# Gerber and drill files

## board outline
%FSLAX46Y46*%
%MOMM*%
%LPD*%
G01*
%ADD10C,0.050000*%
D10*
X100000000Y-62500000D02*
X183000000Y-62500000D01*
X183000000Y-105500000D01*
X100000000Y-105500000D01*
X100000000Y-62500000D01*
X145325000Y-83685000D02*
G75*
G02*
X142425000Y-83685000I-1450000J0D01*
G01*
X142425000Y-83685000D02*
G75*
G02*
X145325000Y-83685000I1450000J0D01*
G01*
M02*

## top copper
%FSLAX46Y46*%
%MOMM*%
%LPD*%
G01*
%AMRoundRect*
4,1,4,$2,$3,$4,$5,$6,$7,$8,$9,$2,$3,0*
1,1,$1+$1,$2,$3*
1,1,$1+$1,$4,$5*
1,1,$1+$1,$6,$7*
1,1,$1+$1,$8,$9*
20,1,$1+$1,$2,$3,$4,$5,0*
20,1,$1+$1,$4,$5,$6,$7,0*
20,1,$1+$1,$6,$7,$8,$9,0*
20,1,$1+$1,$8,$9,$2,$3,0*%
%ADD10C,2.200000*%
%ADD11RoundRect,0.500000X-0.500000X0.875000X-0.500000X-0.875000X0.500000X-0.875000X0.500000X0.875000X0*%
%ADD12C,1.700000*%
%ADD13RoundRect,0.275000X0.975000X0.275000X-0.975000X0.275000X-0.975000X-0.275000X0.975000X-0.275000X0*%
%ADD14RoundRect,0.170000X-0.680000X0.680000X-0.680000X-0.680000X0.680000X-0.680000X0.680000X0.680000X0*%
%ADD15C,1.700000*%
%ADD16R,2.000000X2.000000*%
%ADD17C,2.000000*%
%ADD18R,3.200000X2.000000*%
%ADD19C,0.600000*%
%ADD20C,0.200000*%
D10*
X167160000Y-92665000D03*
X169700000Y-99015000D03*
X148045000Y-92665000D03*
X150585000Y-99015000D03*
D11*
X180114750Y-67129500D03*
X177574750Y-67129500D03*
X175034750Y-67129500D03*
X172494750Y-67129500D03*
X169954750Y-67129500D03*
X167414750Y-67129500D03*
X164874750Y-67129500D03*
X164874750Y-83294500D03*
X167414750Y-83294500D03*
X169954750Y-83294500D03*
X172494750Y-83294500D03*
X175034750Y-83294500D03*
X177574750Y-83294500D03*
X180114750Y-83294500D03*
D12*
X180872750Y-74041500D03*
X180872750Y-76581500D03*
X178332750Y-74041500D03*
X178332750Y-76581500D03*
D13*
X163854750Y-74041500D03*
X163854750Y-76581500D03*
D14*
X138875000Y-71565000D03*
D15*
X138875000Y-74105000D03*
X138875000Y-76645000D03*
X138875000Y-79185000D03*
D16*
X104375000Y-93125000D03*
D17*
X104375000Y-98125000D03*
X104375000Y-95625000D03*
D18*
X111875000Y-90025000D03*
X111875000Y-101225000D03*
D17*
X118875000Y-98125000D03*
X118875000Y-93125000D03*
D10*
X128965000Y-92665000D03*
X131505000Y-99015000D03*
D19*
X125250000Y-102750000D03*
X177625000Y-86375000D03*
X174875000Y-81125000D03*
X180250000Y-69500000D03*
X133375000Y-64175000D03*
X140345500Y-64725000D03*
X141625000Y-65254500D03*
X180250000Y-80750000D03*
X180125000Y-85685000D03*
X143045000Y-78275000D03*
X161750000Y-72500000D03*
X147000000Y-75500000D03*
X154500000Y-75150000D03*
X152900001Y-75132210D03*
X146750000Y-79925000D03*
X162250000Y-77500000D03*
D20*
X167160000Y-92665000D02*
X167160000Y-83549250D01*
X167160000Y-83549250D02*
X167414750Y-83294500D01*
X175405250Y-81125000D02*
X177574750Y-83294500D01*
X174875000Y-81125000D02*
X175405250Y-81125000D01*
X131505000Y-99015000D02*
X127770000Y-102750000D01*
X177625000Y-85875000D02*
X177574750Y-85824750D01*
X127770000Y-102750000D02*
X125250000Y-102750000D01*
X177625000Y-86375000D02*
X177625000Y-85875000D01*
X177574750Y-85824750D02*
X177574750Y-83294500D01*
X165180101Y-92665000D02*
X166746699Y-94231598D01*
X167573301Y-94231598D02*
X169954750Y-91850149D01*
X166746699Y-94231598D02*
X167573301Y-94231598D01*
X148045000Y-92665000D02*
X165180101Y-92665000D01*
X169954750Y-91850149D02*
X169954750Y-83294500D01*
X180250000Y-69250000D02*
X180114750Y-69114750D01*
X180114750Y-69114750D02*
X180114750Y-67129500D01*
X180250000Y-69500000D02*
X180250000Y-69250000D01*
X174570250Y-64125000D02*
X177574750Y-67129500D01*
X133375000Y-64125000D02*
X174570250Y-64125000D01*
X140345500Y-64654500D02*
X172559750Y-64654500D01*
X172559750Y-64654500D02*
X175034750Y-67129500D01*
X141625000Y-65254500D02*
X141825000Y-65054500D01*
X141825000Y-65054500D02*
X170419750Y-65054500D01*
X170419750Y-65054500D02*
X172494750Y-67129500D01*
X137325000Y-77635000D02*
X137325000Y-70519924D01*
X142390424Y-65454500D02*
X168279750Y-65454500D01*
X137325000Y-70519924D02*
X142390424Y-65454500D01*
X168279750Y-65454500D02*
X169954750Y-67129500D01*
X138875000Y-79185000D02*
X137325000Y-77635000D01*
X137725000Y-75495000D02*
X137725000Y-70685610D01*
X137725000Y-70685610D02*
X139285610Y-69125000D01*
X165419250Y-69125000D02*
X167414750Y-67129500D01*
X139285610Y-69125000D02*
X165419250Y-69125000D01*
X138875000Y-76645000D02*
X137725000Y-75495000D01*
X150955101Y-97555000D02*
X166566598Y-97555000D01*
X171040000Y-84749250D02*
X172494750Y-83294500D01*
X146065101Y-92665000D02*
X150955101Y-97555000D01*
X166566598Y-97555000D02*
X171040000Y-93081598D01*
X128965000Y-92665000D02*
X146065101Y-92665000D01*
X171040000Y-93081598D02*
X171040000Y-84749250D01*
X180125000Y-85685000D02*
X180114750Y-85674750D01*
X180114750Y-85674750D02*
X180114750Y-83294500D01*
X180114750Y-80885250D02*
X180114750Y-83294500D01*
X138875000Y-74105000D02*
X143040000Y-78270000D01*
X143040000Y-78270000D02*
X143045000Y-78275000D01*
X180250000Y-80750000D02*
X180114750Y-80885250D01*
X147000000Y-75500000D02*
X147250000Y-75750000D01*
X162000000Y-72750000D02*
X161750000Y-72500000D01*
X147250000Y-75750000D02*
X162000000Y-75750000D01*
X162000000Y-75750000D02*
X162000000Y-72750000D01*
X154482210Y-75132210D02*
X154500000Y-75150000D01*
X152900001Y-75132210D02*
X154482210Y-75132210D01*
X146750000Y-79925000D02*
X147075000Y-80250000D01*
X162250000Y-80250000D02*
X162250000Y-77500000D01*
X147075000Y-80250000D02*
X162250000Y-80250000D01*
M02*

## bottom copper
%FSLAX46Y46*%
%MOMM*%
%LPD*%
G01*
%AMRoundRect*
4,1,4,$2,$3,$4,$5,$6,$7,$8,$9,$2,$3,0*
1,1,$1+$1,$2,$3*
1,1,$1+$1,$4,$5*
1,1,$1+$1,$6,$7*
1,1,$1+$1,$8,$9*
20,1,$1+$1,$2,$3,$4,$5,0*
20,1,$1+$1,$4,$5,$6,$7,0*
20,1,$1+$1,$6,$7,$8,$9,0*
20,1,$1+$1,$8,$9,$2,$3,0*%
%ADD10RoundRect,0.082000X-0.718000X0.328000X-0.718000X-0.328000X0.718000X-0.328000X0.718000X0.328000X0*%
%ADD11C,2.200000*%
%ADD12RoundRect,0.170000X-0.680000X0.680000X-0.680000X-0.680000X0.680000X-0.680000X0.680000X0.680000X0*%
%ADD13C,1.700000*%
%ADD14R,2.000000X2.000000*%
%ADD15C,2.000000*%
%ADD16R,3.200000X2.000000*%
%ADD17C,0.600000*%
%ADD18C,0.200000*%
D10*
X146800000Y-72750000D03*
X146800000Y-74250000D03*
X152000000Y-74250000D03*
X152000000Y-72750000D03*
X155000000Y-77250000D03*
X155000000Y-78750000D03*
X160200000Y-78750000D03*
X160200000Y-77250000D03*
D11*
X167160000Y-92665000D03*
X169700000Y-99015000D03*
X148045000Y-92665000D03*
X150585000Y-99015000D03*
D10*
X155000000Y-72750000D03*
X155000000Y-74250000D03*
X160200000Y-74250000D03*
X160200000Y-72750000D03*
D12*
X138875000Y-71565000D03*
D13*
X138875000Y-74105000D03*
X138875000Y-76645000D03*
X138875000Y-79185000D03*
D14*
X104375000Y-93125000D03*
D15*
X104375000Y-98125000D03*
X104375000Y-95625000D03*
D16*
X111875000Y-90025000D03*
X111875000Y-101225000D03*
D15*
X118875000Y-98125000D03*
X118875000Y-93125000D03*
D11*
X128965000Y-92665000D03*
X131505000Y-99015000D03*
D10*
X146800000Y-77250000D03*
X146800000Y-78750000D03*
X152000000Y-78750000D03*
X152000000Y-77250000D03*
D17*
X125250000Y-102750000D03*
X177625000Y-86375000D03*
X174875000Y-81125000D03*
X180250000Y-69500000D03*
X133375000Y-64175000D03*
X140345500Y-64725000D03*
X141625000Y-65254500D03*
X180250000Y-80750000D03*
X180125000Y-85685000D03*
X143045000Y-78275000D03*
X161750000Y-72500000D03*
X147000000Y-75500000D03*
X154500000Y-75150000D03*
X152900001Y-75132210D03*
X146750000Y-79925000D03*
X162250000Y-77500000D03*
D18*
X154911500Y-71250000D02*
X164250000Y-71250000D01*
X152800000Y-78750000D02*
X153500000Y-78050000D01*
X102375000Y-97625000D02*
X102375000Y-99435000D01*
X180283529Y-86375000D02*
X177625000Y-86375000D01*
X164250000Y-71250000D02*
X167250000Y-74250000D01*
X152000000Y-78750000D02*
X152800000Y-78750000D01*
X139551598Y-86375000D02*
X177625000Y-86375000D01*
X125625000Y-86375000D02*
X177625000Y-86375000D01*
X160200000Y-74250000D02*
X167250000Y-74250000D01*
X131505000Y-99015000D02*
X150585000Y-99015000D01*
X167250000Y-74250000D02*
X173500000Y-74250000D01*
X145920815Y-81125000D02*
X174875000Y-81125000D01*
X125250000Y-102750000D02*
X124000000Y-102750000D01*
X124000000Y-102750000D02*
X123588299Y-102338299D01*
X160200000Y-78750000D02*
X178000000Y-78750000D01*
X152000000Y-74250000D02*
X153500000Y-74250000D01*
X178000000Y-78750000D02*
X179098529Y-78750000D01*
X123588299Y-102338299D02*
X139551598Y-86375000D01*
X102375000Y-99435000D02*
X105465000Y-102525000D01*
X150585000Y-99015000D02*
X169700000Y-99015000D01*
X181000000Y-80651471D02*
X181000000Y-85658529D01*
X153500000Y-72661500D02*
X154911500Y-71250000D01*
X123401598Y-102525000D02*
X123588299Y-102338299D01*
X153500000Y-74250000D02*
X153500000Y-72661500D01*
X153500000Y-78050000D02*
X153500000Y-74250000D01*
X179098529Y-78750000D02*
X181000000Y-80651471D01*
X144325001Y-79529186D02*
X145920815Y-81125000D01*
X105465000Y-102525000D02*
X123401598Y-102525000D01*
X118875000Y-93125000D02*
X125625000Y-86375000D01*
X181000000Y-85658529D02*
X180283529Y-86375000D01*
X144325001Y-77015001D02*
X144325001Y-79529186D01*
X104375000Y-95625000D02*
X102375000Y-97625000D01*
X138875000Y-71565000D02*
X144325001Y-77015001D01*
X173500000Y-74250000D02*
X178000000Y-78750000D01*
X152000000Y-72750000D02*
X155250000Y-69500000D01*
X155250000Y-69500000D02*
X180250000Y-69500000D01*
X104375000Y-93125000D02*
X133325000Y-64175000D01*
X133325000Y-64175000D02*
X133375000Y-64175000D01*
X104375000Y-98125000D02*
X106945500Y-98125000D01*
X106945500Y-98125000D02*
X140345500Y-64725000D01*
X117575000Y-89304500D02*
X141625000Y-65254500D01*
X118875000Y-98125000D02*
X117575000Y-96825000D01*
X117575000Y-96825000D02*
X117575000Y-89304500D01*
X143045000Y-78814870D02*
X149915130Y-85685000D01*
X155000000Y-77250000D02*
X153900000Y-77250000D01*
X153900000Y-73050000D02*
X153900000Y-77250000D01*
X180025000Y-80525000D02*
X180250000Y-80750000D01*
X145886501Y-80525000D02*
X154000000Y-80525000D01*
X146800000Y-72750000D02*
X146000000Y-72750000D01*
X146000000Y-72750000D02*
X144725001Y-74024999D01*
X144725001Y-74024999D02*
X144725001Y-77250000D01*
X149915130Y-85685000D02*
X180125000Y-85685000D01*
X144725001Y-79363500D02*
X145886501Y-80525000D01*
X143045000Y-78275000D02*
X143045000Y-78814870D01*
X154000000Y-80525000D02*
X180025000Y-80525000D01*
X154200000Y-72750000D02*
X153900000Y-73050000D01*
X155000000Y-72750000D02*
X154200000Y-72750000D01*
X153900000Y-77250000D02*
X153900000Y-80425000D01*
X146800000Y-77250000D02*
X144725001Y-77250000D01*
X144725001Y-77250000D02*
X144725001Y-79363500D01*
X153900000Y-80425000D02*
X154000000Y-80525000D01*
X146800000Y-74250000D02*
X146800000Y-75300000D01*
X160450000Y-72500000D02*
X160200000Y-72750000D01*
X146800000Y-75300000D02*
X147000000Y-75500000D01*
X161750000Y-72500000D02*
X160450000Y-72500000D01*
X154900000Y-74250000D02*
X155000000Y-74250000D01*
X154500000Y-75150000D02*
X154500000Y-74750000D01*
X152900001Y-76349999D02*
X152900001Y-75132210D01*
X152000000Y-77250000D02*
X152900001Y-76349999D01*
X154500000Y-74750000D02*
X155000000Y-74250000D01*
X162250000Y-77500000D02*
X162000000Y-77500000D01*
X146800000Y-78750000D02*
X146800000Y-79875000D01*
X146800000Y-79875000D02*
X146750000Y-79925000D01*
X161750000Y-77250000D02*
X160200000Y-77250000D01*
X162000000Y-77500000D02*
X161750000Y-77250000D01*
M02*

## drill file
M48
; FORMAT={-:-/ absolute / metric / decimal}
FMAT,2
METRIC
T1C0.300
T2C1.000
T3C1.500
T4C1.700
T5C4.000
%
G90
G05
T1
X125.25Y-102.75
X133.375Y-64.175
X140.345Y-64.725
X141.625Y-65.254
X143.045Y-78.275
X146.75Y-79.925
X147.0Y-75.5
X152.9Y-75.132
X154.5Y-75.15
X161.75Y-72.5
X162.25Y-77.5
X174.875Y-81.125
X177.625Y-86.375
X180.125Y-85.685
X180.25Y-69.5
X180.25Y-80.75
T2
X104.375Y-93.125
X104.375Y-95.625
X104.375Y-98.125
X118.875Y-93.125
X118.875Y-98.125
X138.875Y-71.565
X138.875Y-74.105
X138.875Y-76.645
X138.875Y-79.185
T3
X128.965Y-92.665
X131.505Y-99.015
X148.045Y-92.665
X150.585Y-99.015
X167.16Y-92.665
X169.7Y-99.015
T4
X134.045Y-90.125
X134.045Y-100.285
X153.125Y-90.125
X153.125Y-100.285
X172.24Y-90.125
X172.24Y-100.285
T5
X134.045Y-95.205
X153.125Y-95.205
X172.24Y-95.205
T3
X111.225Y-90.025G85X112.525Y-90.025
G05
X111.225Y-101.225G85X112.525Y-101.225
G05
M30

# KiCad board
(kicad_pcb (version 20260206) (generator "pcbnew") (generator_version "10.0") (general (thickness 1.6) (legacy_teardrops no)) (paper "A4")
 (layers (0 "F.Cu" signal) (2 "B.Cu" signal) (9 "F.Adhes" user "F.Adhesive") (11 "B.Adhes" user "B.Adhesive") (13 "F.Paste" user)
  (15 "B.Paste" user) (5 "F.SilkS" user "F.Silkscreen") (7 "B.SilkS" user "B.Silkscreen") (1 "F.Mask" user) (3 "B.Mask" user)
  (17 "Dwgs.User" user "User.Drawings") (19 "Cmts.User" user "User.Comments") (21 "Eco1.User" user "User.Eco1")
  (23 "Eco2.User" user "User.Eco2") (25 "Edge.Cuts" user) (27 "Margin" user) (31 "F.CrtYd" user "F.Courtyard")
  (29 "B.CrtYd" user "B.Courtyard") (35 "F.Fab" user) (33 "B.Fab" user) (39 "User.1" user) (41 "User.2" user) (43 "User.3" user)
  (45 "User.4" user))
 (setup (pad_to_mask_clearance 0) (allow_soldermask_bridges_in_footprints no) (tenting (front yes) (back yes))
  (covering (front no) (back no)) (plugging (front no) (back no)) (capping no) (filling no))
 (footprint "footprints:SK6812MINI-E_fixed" (layer "F.Cu") (at 149.399999 73.602842)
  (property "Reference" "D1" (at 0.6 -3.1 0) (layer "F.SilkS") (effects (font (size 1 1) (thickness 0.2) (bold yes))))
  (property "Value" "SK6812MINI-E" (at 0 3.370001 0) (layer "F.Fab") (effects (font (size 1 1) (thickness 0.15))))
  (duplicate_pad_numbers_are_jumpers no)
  (pad "1" smd roundrect (at -2.599999 -0.852842 270) (size 0.82 1.6) (layers "B.Cu" "B.Mask" "B.Paste") (roundrect_rratio 0.1) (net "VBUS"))
  (pad "2" smd roundrect (at -2.599999 0.647158 270) (size 0.82 1.6) (layers "B.Cu" "B.Mask" "B.Paste") (roundrect_rratio 0.1)
   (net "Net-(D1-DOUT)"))
  (pad "3" smd roundrect (at 2.600001 0.647158 270) (size 0.82 1.6) (layers "B.Cu" "B.Mask" "B.Paste") (roundrect_rratio 0.1) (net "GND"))
  (pad "4" smd roundrect (at 2.600001 -0.852842 270) (size 0.82 1.6) (layers "B.Cu" "B.Mask" "B.Paste") (roundrect_rratio 0.1)
   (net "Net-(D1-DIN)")))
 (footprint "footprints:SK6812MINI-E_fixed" (layer "F.Cu") (at 157.599999 78.102842)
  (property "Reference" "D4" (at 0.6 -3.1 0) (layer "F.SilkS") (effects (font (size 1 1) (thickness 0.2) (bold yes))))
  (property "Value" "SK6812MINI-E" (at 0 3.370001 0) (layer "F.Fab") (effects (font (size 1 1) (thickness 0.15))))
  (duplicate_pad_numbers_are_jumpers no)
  (pad "1" smd roundrect (at -2.599999 -0.852842 270) (size 0.82 1.6) (layers "B.Cu" "B.Mask" "B.Paste") (roundrect_rratio 0.1) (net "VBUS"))
  (pad "2" smd roundrect (at -2.599999 0.647158 270) (size 0.82 1.6) (layers "B.Cu" "B.Mask" "B.Paste") (roundrect_rratio 0.1)
   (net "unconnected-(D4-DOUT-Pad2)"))
  (pad "3" smd roundrect (at 2.600001 0.647158 270) (size 0.82 1.6) (layers "B.Cu" "B.Mask" "B.Paste") (roundrect_rratio 0.1) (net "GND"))
  (pad "4" smd roundrect (at 2.600001 -0.852842 270) (size 0.82 1.6) (layers "B.Cu" "B.Mask" "B.Paste") (roundrect_rratio 0.1)
   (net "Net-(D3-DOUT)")))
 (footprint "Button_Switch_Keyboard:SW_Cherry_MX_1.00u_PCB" (layer "F.Cu") (at 167.16 92.665 90)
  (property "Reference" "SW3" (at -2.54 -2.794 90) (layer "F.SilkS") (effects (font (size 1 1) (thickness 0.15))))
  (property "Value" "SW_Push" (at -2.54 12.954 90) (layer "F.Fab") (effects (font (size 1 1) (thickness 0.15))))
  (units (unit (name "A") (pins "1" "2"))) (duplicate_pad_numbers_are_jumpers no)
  (pad "" np_thru_hole circle (at -7.62 5.08 90) (size 1.7 1.7) (drill 1.7) (layers "*.Cu" "*.Mask"))
  (pad "" np_thru_hole circle (at -2.54 5.08 90) (size 4 4) (drill 4) (layers "*.Cu" "*.Mask"))
  (pad "" np_thru_hole circle (at 2.54 5.08 90) (size 1.7 1.7) (drill 1.7) (layers "*.Cu" "*.Mask"))
  (pad "1" thru_hole circle (at 0 0 90) (size 2.2 2.2) (drill 1.5) (layers "*.Cu" "*.Mask") (remove_unused_layers no) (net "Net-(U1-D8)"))
  (pad "2" thru_hole circle (at -6.35 2.54 90) (size 2.2 2.2) (drill 1.5) (layers "*.Cu" "*.Mask") (remove_unused_layers no) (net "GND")))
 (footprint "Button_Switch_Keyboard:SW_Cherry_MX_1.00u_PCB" (layer "F.Cu") (at 148.045 92.665 90)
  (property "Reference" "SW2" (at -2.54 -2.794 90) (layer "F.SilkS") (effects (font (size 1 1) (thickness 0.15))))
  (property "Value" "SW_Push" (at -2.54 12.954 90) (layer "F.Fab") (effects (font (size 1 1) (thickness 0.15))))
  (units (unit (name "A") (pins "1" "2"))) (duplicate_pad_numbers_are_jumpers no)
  (pad "" np_thru_hole circle (at -7.62 5.08 90) (size 1.7 1.7) (drill 1.7) (layers "*.Cu" "*.Mask"))
  (pad "" np_thru_hole circle (at -2.54 5.08 90) (size 4 4) (drill 4) (layers "*.Cu" "*.Mask"))
  (pad "" np_thru_hole circle (at 2.54 5.08 90) (size 1.7 1.7) (drill 1.7) (layers "*.Cu" "*.Mask"))
  (pad "1" thru_hole circle (at 0 0 90) (size 2.2 2.2) (drill 1.5) (layers "*.Cu" "*.Mask") (remove_unused_layers no) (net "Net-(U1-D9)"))
  (pad "2" thru_hole circle (at -6.35 2.54 90) (size 2.2 2.2) (drill 1.5) (layers "*.Cu" "*.Mask") (remove_unused_layers no) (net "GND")))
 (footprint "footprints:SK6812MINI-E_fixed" (layer "F.Cu") (at 157.599999 73.602842)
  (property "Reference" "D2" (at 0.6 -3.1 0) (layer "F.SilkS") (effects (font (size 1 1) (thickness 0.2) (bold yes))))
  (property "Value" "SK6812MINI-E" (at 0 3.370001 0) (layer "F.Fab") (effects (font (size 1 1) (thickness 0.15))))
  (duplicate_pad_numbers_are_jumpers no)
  (pad "1" smd roundrect (at -2.599999 -0.852842 270) (size 0.82 1.6) (layers "B.Cu" "B.Mask" "B.Paste") (roundrect_rratio 0.1) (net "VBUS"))
  (pad "2" smd roundrect (at -2.599999 0.647158 270) (size 0.82 1.6) (layers "B.Cu" "B.Mask" "B.Paste") (roundrect_rratio 0.1)
   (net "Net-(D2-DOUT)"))
  (pad "3" smd roundrect (at 2.600001 0.647158 270) (size 0.82 1.6) (layers "B.Cu" "B.Mask" "B.Paste") (roundrect_rratio 0.1) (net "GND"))
  (pad "4" smd roundrect (at 2.600001 -0.852842 270) (size 0.82 1.6) (layers "B.Cu" "B.Mask" "B.Paste") (roundrect_rratio 0.1)
   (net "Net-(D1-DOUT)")))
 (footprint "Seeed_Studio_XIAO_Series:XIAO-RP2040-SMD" (layer "F.Cu") (at 161.99475 66.2945 -90)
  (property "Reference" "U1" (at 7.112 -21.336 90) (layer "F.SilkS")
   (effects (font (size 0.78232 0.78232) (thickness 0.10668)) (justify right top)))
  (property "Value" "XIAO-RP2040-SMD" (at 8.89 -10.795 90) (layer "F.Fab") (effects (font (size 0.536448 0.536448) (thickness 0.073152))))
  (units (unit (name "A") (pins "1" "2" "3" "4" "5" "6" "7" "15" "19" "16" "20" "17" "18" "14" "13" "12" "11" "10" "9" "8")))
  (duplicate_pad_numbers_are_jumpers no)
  (pad "1" smd roundrect (at 0.835 -18.12 270) (size 2.75 2) (layers "F.Cu" "F.Mask" "F.Paste") (roundrect_rratio 0.25) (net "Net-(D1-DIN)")
   (solder_mask_margin 0.0508) (thermal_bridge_angle 45))
  (pad "2" smd roundrect (at 0.835 -15.58 270) (size 2.75 2) (layers "F.Cu" "F.Mask" "F.Paste") (roundrect_rratio 0.25) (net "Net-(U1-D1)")
   (solder_mask_margin 0.0508) (thermal_bridge_angle 45))
  (pad "3" smd roundrect (at 0.835 -13.04 270) (size 2.75 2) (layers "F.Cu" "F.Mask" "F.Paste") (roundrect_rratio 0.25) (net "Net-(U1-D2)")
   (solder_mask_margin 0.0508) (thermal_bridge_angle 45))
  (pad "4" smd roundrect (at 0.835 -10.5 270) (size 2.75 2) (layers "F.Cu" "F.Mask" "F.Paste") (roundrect_rratio 0.25) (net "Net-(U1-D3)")
   (solder_mask_margin 0.0508) (thermal_bridge_angle 45))
  (pad "5" smd roundrect (at 0.835 -7.96 270) (size 2.75 2) (layers "F.Cu" "F.Mask" "F.Paste") (roundrect_rratio 0.25) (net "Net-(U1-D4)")
   (solder_mask_margin 0.0508) (thermal_bridge_angle 45))
  (pad "6" smd roundrect (at 0.835 -5.42 270) (size 2.75 2) (layers "F.Cu" "F.Mask" "F.Paste") (roundrect_rratio 0.25) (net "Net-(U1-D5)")
   (solder_mask_margin 0.0508) (thermal_bridge_angle 45))
  (pad "7" smd roundrect (at 0.835 -2.88 270) (size 2.75 2) (layers "F.Cu" "F.Mask" "F.Paste") (roundrect_rratio 0.25)
   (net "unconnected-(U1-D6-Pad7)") (solder_mask_margin 0.0508) (thermal_bridge_angle 45))
  (pad "8" smd roundrect (at 17 -2.88 270) (size 2.75 2) (layers "F.Cu" "F.Mask" "F.Paste") (roundrect_rratio 0.25)
   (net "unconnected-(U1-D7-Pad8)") (solder_mask_margin 0.0508) (thermal_bridge_angle 45))
  (pad "9" smd roundrect (at 17 -5.42 270) (size 2.75 2) (layers "F.Cu" "F.Mask" "F.Paste") (roundrect_rratio 0.25) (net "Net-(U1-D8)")
   (solder_mask_margin 0.0508) (thermal_bridge_angle 45))
  (pad "10" smd roundrect (at 17 -7.96 270) (size 2.75 2) (layers "F.Cu" "F.Mask" "F.Paste") (roundrect_rratio 0.25) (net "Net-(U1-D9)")
   (solder_mask_margin 0.0508) (thermal_bridge_angle 45))
  (pad "11" smd roundrect (at 17 -10.5 270) (size 2.75 2) (layers "F.Cu" "F.Mask" "F.Paste") (roundrect_rratio 0.25) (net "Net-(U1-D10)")
   (solder_mask_margin 0.0508) (thermal_bridge_angle 45))
  (pad "12" smd roundrect (at 17 -13.04 270) (size 2.75 2) (layers "F.Cu" "F.Mask" "F.Paste") (roundrect_rratio 0.25)
   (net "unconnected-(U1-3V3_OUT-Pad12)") (solder_mask_margin 0.0508) (thermal_bridge_angle 45))
  (pad "13" smd roundrect (at 17 -15.58 270) (size 2.75 2) (layers "F.Cu" "F.Mask" "F.Paste") (roundrect_rratio 0.25) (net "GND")
   (solder_mask_margin 0.0508) (thermal_bridge_angle 45))
  (pad "14" smd roundrect (at 17 -18.12 270) (size 2.75 2) (layers "F.Cu" "F.Mask" "F.Paste") (roundrect_rratio 0.25) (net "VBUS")
   (solder_mask_margin 0.0508) (thermal_bridge_angle 45))
  (pad "15" smd circle (at 7.747 -18.878 270) (size 1.7 1.7) (layers "F.Cu" "F.Mask" "F.Paste") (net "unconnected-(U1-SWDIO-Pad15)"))
  (pad "16" smd circle (at 10.287 -18.878 270) (size 1.7 1.7) (layers "F.Cu" "F.Mask" "F.Paste") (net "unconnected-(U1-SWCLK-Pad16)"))
  (pad "17" smd circle (at 7.747 -16.338 270) (size 1.7 1.7) (layers "F.Cu" "F.Mask" "F.Paste") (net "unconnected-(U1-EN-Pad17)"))
  (pad "18" smd circle (at 10.287 -16.338 270) (size 1.7 1.7) (layers "F.Cu" "F.Mask" "F.Paste") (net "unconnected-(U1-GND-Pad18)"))
  (pad "19" smd roundrect (at 7.747 -1.86 180) (size 2.5 1.1) (layers "F.Cu" "F.Mask" "F.Paste") (roundrect_rratio 0.25)
   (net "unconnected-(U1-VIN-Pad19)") (thermal_bridge_angle 45))
  (pad "20" smd roundrect (at 10.287 -1.86 180) (size 2.5 1.1) (layers "F.Cu" "F.Mask" "F.Paste") (roundrect_rratio 0.25)
   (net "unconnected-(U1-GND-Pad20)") (thermal_bridge_angle 45)))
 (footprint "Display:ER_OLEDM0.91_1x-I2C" (layer "F.Cu") (at 138.875 71.565 -90)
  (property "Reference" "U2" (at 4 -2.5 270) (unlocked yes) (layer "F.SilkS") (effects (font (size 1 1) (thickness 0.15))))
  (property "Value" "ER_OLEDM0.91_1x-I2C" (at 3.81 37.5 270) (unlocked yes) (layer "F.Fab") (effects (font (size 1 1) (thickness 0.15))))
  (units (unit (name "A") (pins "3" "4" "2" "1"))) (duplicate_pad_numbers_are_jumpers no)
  (pad "1" thru_hole roundrect (at 0 0 270) (size 1.7 1.7) (drill 1) (layers "*.Cu" "*.Mask") (remove_unused_layers no)
   (roundrect_rratio 0.1) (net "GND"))
  (pad "2" thru_hole circle (at 2.54 0 270) (size 1.7 1.7) (drill 1) (layers "*.Cu" "*.Mask") (remove_unused_layers no) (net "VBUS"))
  (pad "3" thru_hole circle (at 5.08 0 270) (size 1.7 1.7) (drill 1) (layers "*.Cu" "*.Mask") (remove_unused_layers no) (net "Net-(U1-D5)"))
  (pad "4" thru_hole circle (at 7.62 0 270) (size 1.7 1.7) (drill 1) (layers "*.Cu" "*.Mask") (remove_unused_layers no) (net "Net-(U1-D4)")))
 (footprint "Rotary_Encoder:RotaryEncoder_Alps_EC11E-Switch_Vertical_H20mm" (layer "F.Cu") (at 104.375 93.125)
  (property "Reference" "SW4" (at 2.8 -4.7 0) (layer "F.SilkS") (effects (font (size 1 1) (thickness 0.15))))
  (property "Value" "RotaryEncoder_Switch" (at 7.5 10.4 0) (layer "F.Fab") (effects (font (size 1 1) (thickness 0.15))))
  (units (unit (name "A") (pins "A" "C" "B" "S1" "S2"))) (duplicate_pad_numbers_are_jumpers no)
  (pad "A" thru_hole rect (at 0 0) (size 2 2) (drill 1) (layers "*.Cu" "*.Mask") (remove_unused_layers no) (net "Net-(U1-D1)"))
  (pad "B" thru_hole circle (at 0 5) (size 2 2) (drill 1) (layers "*.Cu" "*.Mask") (remove_unused_layers no) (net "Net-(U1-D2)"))
  (pad "C" thru_hole circle (at 0 2.5) (size 2 2) (drill 1) (layers "*.Cu" "*.Mask") (remove_unused_layers no) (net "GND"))
  (pad "MP" thru_hole rect (at 7.5 -3.1) (size 3.2 2) (drill oval 2.8 1.5) (layers "*.Cu" "*.Mask") (remove_unused_layers no))
  (pad "MP" thru_hole rect (at 7.5 8.1) (size 3.2 2) (drill oval 2.8 1.5) (layers "*.Cu" "*.Mask") (remove_unused_layers no))
  (pad "S1" thru_hole circle (at 14.5 5) (size 2 2) (drill 1) (layers "*.Cu" "*.Mask") (remove_unused_layers no) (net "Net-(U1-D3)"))
  (pad "S2" thru_hole circle (at 14.5 0) (size 2 2) (drill 1) (layers "*.Cu" "*.Mask") (remove_unused_layers no) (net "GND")))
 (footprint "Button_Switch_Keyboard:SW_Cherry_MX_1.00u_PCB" (layer "F.Cu") (at 128.965 92.665 90)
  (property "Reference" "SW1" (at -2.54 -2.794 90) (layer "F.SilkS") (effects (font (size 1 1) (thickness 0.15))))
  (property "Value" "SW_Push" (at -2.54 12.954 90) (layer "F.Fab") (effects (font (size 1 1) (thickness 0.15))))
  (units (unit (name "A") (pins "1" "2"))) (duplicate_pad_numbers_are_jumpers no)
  (pad "" np_thru_hole circle (at -7.62 5.08 90) (size 1.7 1.7) (drill 1.7) (layers "*.Cu" "*.Mask"))
  (pad "" np_thru_hole circle (at -2.54 5.08 90) (size 4 4) (drill 4) (layers "*.Cu" "*.Mask"))
  (pad "" np_thru_hole circle (at 2.54 5.08 90) (size 1.7 1.7) (drill 1.7) (layers "*.Cu" "*.Mask"))
  (pad "1" thru_hole circle (at 0 0 90) (size 2.2 2.2) (drill 1.5) (layers "*.Cu" "*.Mask") (remove_unused_layers no) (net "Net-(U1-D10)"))
  (pad "2" thru_hole circle (at -6.35 2.54 90) (size 2.2 2.2) (drill 1.5) (layers "*.Cu" "*.Mask") (remove_unused_layers no) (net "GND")))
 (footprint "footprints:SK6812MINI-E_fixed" (layer "F.Cu") (at 149.399999 78.102842)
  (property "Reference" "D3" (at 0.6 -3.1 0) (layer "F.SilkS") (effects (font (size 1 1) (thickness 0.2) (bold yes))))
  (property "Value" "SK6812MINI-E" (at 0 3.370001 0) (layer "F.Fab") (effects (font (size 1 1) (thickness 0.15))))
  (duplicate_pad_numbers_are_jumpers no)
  (pad "1" smd roundrect (at -2.599999 -0.852842 270) (size 0.82 1.6) (layers "B.Cu" "B.Mask" "B.Paste") (roundrect_rratio 0.1) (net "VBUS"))
  (pad "2" smd roundrect (at -2.599999 0.647158 270) (size 0.82 1.6) (layers "B.Cu" "B.Mask" "B.Paste") (roundrect_rratio 0.1)
   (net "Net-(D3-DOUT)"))
  (pad "3" smd roundrect (at 2.600001 0.647158 270) (size 0.82 1.6) (layers "B.Cu" "B.Mask" "B.Paste") (roundrect_rratio 0.1) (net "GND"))
  (pad "4" smd roundrect (at 2.600001 -0.852842 270) (size 0.82 1.6) (layers "B.Cu" "B.Mask" "B.Paste") (roundrect_rratio 0.1)
   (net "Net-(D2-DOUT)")))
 (gr_rect (start 100 62.5) (end 183 105.5) (stroke (width 0.05) (type solid)) (fill no) (layer "Edge.Cuts"))
 (gr_circle (center 143.875 83.685) (end 145.325 83.685) (stroke (width 0.05) (type default)) (fill no) (layer "Edge.Cuts"))
 (segment (start 167.16 92.665) (end 167.16 83.54925) (width 0.2) (layer "F.Cu") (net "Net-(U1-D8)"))
 (segment (start 167.16 83.54925) (end 167.41475 83.2945) (width 0.2) (layer "F.Cu") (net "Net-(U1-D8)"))
 (segment (start 175.40525 81.125) (end 177.57475 83.2945) (width 0.2) (layer "F.Cu") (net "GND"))
 (segment (start 174.875 81.125) (end 175.40525 81.125) (width 0.2) (layer "F.Cu") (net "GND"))
 (segment (start 131.505 99.015) (end 127.77 102.75) (width 0.2) (layer "F.Cu") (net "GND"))
 (segment (start 177.625 85.875) (end 177.57475 85.82475) (width 0.2) (layer "F.Cu") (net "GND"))
 (segment (start 127.77 102.75) (end 125.25 102.75) (width 0.2) (layer "F.Cu") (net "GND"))
 (segment (start 177.625 86.375) (end 177.625 85.875) (width 0.2) (layer "F.Cu") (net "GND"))
 (segment (start 177.57475 85.82475) (end 177.57475 83.2945) (width 0.2) (layer "F.Cu") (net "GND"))
 (via (at 125.25 102.75) (size 0.6) (drill 0.3) (layers "F.Cu" "B.Cu") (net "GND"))
 (via (at 177.625 86.375) (size 0.6) (drill 0.3) (layers "F.Cu" "B.Cu") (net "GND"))
 (via (at 174.875 81.125) (size 0.6) (drill 0.3) (layers "F.Cu" "B.Cu") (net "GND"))
 (segment (start 154.9115 71.25) (end 164.25 71.25) (width 0.2) (layer "B.Cu") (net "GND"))
 (segment (start 152.8 78.75) (end 153.5 78.05) (width 0.2) (layer "B.Cu") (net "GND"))
 (segment (start 102.375 97.625) (end 102.375 99.435) (width 0.2) (layer "B.Cu") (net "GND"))
 (segment (start 180.283529 86.375) (end 177.625 86.375) (width 0.2) (layer "B.Cu") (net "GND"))
 (segment (start 164.25 71.25) (end 167.25 74.25) (width 0.2) (layer "B.Cu") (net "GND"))
 (segment (start 152 78.75) (end 152.8 78.75) (width 0.2) (layer "B.Cu") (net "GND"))
 (segment (start 139.551598 86.375) (end 177.625 86.375) (width 0.2) (layer "B.Cu") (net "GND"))
 (segment (start 125.625 86.375) (end 177.625 86.375) (width 0.2) (layer "B.Cu") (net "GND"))
 (segment (start 160.2 74.25) (end 167.25 74.25) (width 0.2) (layer "B.Cu") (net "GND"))
 (segment (start 131.505 99.015) (end 150.585 99.015) (width 0.2) (layer "B.Cu") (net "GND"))
 (segment (start 167.25 74.25) (end 173.5 74.25) (width 0.2) (layer "B.Cu") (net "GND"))
 (segment (start 145.920815 81.125) (end 174.875 81.125) (width 0.2) (layer "B.Cu") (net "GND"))
 (segment (start 125.25 102.75) (end 124 102.75) (width 0.2) (layer "B.Cu") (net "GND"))
 (segment (start 124 102.75) (end 123.588299 102.338299) (width 0.2) (layer "B.Cu") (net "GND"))
 (segment (start 160.2 78.75) (end 178 78.75) (width 0.2) (layer "B.Cu") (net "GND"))
 (segment (start 152 74.25) (end 153.5 74.25) (width 0.2) (layer "B.Cu") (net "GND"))
 (segment (start 178 78.75) (end 179.098529 78.75) (width 0.2) (layer "B.Cu") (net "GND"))
 (segment (start 123.588299 102.338299) (end 139.551598 86.375) (width 0.2) (layer "B.Cu") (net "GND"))
 (segment (start 102.375 99.435) (end 105.465 102.525) (width 0.2) (layer "B.Cu") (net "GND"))
 (segment (start 150.585 99.015) (end 169.7 99.015) (width 0.2) (layer "B.Cu") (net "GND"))
 (segment (start 181 80.651471) (end 181 85.658529) (width 0.2) (layer "B.Cu") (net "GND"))
 (segment (start 153.5 72.6615) (end 154.9115 71.25) (width 0.2) (layer "B.Cu") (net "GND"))
 (segment (start 123.401598 102.525) (end 123.588299 102.338299) (width 0.2) (layer "B.Cu") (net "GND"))
 (segment (start 153.5 74.25) (end 153.5 72.6615) (width 0.2) (layer "B.Cu") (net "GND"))
 (segment (start 153.5 78.05) (end 153.5 74.25) (width 0.2) (layer "B.Cu") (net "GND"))
 (segment (start 179.098529 78.75) (end 181 80.651471) (width 0.2) (layer "B.Cu") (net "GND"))
 (segment (start 144.325001 79.529186) (end 145.920815 81.125) (width 0.2) (layer "B.Cu") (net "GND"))
 (segment (start 105.465 102.525) (end 123.401598 102.525) (width 0.2) (layer "B.Cu") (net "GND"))
 (segment (start 118.875 93.125) (end 125.625 86.375) (width 0.2) (layer "B.Cu") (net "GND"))
 (segment (start 181 85.658529) (end 180.283529 86.375) (width 0.2) (layer "B.Cu") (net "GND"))
 (segment (start 144.325001 77.015001) (end 144.325001 79.529186) (width 0.2) (layer "B.Cu") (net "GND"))
 (segment (start 104.375 95.625) (end 102.375 97.625) (width 0.2) (layer "B.Cu") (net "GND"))
 (segment (start 138.875 71.565) (end 144.325001 77.015001) (width 0.2) (layer "B.Cu") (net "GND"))
 (segment (start 173.5 74.25) (end 178 78.75) (width 0.2) (layer "B.Cu") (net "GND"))
 (segment (start 165.180101 92.665) (end 166.746699 94.231598) (width 0.2) (layer "F.Cu") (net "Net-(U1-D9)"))
 (segment (start 167.573301 94.231598) (end 169.95475 91.850149) (width 0.2) (layer "F.Cu") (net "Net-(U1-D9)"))
 (segment (start 166.746699 94.231598) (end 167.573301 94.231598) (width 0.2) (layer "F.Cu") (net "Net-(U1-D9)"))
 (segment (start 148.045 92.665) (end 165.180101 92.665) (width 0.2) (layer "F.Cu") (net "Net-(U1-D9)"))
 (segment (start 169.95475 91.850149) (end 169.95475 83.2945) (width 0.2) (layer "F.Cu") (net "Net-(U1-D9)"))
 (segment (start 180.25 69.25) (end 180.11475 69.11475) (width 0.2) (layer "F.Cu") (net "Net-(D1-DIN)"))
 (segment (start 180.11475 69.11475) (end 180.11475 67.1295) (width 0.2) (layer "F.Cu") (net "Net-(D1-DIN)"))
 (segment (start 180.25 69.5) (end 180.25 69.25) (width 0.2) (layer "F.Cu") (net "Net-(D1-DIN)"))
 (via (at 180.25 69.5) (size 0.6) (drill 0.3) (layers "F.Cu" "B.Cu") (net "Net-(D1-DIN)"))
 (segment (start 152 72.75) (end 155.25 69.5) (width 0.2) (layer "B.Cu") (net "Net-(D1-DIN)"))
 (segment (start 155.25 69.5) (end 180.25 69.5) (width 0.2) (layer "B.Cu") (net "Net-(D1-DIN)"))
 (segment (start 174.57025 64.125) (end 177.57475 67.1295) (width 0.2) (layer "F.Cu") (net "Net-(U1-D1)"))
 (segment (start 133.375 64.125) (end 174.57025 64.125) (width 0.2) (layer "F.Cu") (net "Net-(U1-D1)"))
 (via (at 133.375 64.175) (size 0.6) (drill 0.3) (layers "F.Cu" "B.Cu") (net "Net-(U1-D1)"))
 (segment (start 104.375 93.125) (end 133.325 64.175) (width 0.2) (layer "B.Cu") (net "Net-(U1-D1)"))
 (segment (start 133.325 64.175) (end 133.375 64.175) (width 0.2) (layer "B.Cu") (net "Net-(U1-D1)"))
 (segment (start 140.3455 64.6545) (end 172.55975 64.6545) (width 0.2) (layer "F.Cu") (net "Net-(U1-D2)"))
 (segment (start 172.55975 64.6545) (end 175.03475 67.1295) (width 0.2) (layer "F.Cu") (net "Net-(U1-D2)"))
 (via (at 140.3455 64.725) (size 0.6) (drill 0.3) (layers "F.Cu" "B.Cu") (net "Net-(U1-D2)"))
 (segment (start 104.375 98.125) (end 106.9455 98.125) (width 0.2) (layer "B.Cu") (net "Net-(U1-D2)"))
 (segment (start 106.9455 98.125) (end 140.3455 64.725) (width 0.2) (layer "B.Cu") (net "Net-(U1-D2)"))
 (segment (start 141.625 65.2545) (end 141.825 65.0545) (width 0.2) (layer "F.Cu") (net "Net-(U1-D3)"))
 (segment (start 141.825 65.0545) (end 170.41975 65.0545) (width 0.2) (layer "F.Cu") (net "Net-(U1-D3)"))
 (segment (start 170.41975 65.0545) (end 172.49475 67.1295) (width 0.2) (layer "F.Cu") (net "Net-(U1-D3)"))
 (via (at 141.625 65.2545) (size 0.6) (drill 0.3) (layers "F.Cu" "B.Cu") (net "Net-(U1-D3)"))
 (segment (start 117.575 89.3045) (end 141.625 65.2545) (width 0.2) (layer "B.Cu") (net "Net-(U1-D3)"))
 (segment (start 118.875 98.125) (end 117.575 96.825) (width 0.2) (layer "B.Cu") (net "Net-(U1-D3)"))
 (segment (start 117.575 96.825) (end 117.575 89.3045) (width 0.2) (layer "B.Cu") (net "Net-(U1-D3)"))
 (segment (start 137.325 77.635) (end 137.325 70.519924) (width 0.2) (layer "F.Cu") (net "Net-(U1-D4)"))
 (segment (start 142.390424 65.4545) (end 168.27975 65.4545) (width 0.2) (layer "F.Cu") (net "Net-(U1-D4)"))
 (segment (start 137.325 70.519924) (end 142.390424 65.4545) (width 0.2) (layer "F.Cu") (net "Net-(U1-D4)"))
 (segment (start 168.27975 65.4545) (end 169.95475 67.1295) (width 0.2) (layer "F.Cu") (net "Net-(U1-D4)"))
 (segment (start 138.875 79.185) (end 137.325 77.635) (width 0.2) (layer "F.Cu") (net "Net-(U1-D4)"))
 (segment (start 137.725 75.495) (end 137.725 70.68561) (width 0.2) (layer "F.Cu") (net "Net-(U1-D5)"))
 (segment (start 137.725 70.68561) (end 139.28561 69.125) (width 0.2) (layer "F.Cu") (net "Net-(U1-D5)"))
 (segment (start 165.41925 69.125) (end 167.41475 67.1295) (width 0.2) (layer "F.Cu") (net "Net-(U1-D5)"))
 (segment (start 139.28561 69.125) (end 165.41925 69.125) (width 0.2) (layer "F.Cu") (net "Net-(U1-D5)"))
 (segment (start 138.875 76.645) (end 137.725 75.495) (width 0.2) (layer "F.Cu") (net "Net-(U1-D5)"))
 (segment (start 150.955101 97.555) (end 166.566598 97.555) (width 0.2) (layer "F.Cu") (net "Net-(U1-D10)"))
 (segment (start 171.04 84.74925) (end 172.49475 83.2945) (width 0.2) (layer "F.Cu") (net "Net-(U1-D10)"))
 (segment (start 146.065101 92.665) (end 150.955101 97.555) (width 0.2) (layer "F.Cu") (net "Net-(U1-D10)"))
 (segment (start 166.566598 97.555) (end 171.04 93.081598) (width 0.2) (layer "F.Cu") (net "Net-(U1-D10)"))
 (segment (start 128.965 92.665) (end 146.065101 92.665) (width 0.2) (layer "F.Cu") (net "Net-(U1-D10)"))
 (segment (start 171.04 93.081598) (end 171.04 84.74925) (width 0.2) (layer "F.Cu") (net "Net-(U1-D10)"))
 (segment (start 180.125 85.685) (end 180.11475 85.67475) (width 0.2) (layer "F.Cu") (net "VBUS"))
 (segment (start 180.11475 85.67475) (end 180.11475 83.2945) (width 0.2) (layer "F.Cu") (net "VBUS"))
 (segment (start 180.11475 80.88525) (end 180.11475 83.2945) (width 0.2) (layer "F.Cu") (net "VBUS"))
 (segment (start 138.875 74.105) (end 143.04 78.27) (width 0.2) (layer "F.Cu") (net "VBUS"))
 (segment (start 143.04 78.27) (end 143.045 78.275) (width 0.2) (layer "F.Cu") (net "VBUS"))
 (segment (start 180.25 80.75) (end 180.11475 80.88525) (width 0.2) (layer "F.Cu") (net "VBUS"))
 (via (at 180.25 80.75) (size 0.6) (drill 0.3) (layers "F.Cu" "B.Cu") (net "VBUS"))
 (via (at 180.125 85.685) (size 0.6) (drill 0.3) (layers "F.Cu" "B.Cu") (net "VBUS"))
 (via (at 143.045 78.275) (size 0.6) (drill 0.3) (layers "F.Cu" "B.Cu") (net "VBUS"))
 (segment (start 143.045 78.81487) (end 149.91513 85.685) (width 0.2) (layer "B.Cu") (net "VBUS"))
 (segment (start 155 77.25) (end 153.9 77.25) (width 0.2) (layer "B.Cu") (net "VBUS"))
 (segment (start 153.9 73.05) (end 153.9 77.25) (width 0.2) (layer "B.Cu") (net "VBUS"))
 (segment (start 180.025 80.525) (end 180.25 80.75) (width 0.2) (layer "B.Cu") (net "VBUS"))
 (segment (start 145.886501 80.525) (end 154 80.525) (width 0.2) (layer "B.Cu") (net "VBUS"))
 (segment (start 146.8 72.75) (end 146 72.75) (width 0.2) (layer "B.Cu") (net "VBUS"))
 (segment (start 146 72.75) (end 144.725001 74.024999) (width 0.2) (layer "B.Cu") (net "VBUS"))
 (segment (start 144.725001 74.024999) (end 144.725001 77.25) (width 0.2) (layer "B.Cu") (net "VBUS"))
 (segment (start 149.91513 85.685) (end 180.125 85.685) (width 0.2) (layer "B.Cu") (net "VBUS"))
 (segment (start 144.725001 79.3635) (end 145.886501 80.525) (width 0.2) (layer "B.Cu") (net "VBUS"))
 (segment (start 143.045 78.275) (end 143.045 78.81487) (width 0.2) (layer "B.Cu") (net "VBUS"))
 (segment (start 154 80.525) (end 180.025 80.525) (width 0.2) (layer "B.Cu") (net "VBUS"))
 (segment (start 154.2 72.75) (end 153.9 73.05) (width 0.2) (layer "B.Cu") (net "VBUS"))
 (segment (start 155 72.75) (end 154.2 72.75) (width 0.2) (layer "B.Cu") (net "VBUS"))
 (segment (start 153.9 77.25) (end 153.9 80.425) (width 0.2) (layer "B.Cu") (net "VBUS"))
 (segment (start 146.8 77.25) (end 144.725001 77.25) (width 0.2) (layer "B.Cu") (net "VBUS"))
 (segment (start 144.725001 77.25) (end 144.725001 79.3635) (width 0.2) (layer "B.Cu") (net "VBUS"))
 (segment (start 153.9 80.425) (end 154 80.525) (width 0.2) (layer "B.Cu") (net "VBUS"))
 (segment (start 147 75.5) (end 147.25 75.75) (width 0.2) (layer "F.Cu") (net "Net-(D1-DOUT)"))
 (segment (start 162 72.75) (end 161.75 72.5) (width 0.2) (layer "F.Cu") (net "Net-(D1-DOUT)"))
 (segment (start 147.25 75.75) (end 162 75.75) (width 0.2) (layer "F.Cu") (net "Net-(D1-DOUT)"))
 (segment (start 162 75.75) (end 162 72.75) (width 0.2) (layer "F.Cu") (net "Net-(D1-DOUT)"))
 (via (at 161.75 72.5) (size 0.6) (drill 0.3) (layers "F.Cu" "B.Cu") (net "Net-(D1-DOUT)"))
 (via (at 147 75.5) (size 0.6) (drill 0.3) (layers "F.Cu" "B.Cu") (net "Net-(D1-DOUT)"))
 (segment (start 146.8 74.25) (end 146.8 75.3) (width 0.2) (layer "B.Cu") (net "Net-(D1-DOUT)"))
 (segment (start 160.45 72.5) (end 160.2 72.75) (width 0.2) (layer "B.Cu") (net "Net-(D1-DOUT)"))
 (segment (start 146.8 75.3) (end 147 75.5) (width 0.2) (layer "B.Cu") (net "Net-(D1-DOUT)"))
 (segment (start 161.75 72.5) (end 160.45 72.5) (width 0.2) (layer "B.Cu") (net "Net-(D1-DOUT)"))
 (segment (start 154.48221 75.13221) (end 154.5 75.15) (width 0.2) (layer "F.Cu") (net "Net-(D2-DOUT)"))
 (segment (start 152.900001 75.13221) (end 154.48221 75.13221) (width 0.2) (layer "F.Cu") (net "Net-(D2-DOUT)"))
 (via (at 154.5 75.15) (size 0.6) (drill 0.3) (layers "F.Cu" "B.Cu") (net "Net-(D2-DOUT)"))
 (via (at 152.900001 75.13221) (size 0.6) (drill 0.3) (layers "F.Cu" "B.Cu") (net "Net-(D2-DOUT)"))
 (segment (start 154.9 74.25) (end 155 74.25) (width 0.2) (layer "B.Cu") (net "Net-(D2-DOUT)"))
 (segment (start 154.5 75.15) (end 154.5 74.75) (width 0.2) (layer "B.Cu") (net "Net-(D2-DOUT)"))
 (segment (start 152.900001 76.349999) (end 152.900001 75.13221) (width 0.2) (layer "B.Cu") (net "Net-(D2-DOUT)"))
 (segment (start 152 77.25) (end 152.900001 76.349999) (width 0.2) (layer "B.Cu") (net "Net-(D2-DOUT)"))
 (segment (start 154.5 74.75) (end 155 74.25) (width 0.2) (layer "B.Cu") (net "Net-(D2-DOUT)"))
 (segment (start 146.75 79.925) (end 147.075 80.25) (width 0.2) (layer "F.Cu") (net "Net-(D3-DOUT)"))
 (segment (start 162.25 80.25) (end 162.25 77.5) (width 0.2) (layer "F.Cu") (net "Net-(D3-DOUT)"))
 (segment (start 147.075 80.25) (end 162.25 80.25) (width 0.2) (layer "F.Cu") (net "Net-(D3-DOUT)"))
 (via (at 146.75 79.925) (size 0.6) (drill 0.3) (layers "F.Cu" "B.Cu") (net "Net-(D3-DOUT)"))
 (via (at 162.25 77.5) (size 0.6) (drill 0.3) (layers "F.Cu" "B.Cu") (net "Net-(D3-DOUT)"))
 (segment (start 162.25 77.5) (end 162 77.5) (width 0.2) (layer "B.Cu") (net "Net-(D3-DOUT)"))
 (segment (start 146.8 78.75) (end 146.8 79.875) (width 0.2) (layer "B.Cu") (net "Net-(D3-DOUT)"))
 (segment (start 146.8 79.875) (end 146.75 79.925) (width 0.2) (layer "B.Cu") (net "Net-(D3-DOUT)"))
 (segment (start 161.75 77.25) (end 160.2 77.25) (width 0.2) (layer "B.Cu") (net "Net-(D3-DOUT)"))
 (segment (start 162 77.5) (end 161.75 77.25) (width 0.2) (layer "B.Cu") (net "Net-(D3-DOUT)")))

